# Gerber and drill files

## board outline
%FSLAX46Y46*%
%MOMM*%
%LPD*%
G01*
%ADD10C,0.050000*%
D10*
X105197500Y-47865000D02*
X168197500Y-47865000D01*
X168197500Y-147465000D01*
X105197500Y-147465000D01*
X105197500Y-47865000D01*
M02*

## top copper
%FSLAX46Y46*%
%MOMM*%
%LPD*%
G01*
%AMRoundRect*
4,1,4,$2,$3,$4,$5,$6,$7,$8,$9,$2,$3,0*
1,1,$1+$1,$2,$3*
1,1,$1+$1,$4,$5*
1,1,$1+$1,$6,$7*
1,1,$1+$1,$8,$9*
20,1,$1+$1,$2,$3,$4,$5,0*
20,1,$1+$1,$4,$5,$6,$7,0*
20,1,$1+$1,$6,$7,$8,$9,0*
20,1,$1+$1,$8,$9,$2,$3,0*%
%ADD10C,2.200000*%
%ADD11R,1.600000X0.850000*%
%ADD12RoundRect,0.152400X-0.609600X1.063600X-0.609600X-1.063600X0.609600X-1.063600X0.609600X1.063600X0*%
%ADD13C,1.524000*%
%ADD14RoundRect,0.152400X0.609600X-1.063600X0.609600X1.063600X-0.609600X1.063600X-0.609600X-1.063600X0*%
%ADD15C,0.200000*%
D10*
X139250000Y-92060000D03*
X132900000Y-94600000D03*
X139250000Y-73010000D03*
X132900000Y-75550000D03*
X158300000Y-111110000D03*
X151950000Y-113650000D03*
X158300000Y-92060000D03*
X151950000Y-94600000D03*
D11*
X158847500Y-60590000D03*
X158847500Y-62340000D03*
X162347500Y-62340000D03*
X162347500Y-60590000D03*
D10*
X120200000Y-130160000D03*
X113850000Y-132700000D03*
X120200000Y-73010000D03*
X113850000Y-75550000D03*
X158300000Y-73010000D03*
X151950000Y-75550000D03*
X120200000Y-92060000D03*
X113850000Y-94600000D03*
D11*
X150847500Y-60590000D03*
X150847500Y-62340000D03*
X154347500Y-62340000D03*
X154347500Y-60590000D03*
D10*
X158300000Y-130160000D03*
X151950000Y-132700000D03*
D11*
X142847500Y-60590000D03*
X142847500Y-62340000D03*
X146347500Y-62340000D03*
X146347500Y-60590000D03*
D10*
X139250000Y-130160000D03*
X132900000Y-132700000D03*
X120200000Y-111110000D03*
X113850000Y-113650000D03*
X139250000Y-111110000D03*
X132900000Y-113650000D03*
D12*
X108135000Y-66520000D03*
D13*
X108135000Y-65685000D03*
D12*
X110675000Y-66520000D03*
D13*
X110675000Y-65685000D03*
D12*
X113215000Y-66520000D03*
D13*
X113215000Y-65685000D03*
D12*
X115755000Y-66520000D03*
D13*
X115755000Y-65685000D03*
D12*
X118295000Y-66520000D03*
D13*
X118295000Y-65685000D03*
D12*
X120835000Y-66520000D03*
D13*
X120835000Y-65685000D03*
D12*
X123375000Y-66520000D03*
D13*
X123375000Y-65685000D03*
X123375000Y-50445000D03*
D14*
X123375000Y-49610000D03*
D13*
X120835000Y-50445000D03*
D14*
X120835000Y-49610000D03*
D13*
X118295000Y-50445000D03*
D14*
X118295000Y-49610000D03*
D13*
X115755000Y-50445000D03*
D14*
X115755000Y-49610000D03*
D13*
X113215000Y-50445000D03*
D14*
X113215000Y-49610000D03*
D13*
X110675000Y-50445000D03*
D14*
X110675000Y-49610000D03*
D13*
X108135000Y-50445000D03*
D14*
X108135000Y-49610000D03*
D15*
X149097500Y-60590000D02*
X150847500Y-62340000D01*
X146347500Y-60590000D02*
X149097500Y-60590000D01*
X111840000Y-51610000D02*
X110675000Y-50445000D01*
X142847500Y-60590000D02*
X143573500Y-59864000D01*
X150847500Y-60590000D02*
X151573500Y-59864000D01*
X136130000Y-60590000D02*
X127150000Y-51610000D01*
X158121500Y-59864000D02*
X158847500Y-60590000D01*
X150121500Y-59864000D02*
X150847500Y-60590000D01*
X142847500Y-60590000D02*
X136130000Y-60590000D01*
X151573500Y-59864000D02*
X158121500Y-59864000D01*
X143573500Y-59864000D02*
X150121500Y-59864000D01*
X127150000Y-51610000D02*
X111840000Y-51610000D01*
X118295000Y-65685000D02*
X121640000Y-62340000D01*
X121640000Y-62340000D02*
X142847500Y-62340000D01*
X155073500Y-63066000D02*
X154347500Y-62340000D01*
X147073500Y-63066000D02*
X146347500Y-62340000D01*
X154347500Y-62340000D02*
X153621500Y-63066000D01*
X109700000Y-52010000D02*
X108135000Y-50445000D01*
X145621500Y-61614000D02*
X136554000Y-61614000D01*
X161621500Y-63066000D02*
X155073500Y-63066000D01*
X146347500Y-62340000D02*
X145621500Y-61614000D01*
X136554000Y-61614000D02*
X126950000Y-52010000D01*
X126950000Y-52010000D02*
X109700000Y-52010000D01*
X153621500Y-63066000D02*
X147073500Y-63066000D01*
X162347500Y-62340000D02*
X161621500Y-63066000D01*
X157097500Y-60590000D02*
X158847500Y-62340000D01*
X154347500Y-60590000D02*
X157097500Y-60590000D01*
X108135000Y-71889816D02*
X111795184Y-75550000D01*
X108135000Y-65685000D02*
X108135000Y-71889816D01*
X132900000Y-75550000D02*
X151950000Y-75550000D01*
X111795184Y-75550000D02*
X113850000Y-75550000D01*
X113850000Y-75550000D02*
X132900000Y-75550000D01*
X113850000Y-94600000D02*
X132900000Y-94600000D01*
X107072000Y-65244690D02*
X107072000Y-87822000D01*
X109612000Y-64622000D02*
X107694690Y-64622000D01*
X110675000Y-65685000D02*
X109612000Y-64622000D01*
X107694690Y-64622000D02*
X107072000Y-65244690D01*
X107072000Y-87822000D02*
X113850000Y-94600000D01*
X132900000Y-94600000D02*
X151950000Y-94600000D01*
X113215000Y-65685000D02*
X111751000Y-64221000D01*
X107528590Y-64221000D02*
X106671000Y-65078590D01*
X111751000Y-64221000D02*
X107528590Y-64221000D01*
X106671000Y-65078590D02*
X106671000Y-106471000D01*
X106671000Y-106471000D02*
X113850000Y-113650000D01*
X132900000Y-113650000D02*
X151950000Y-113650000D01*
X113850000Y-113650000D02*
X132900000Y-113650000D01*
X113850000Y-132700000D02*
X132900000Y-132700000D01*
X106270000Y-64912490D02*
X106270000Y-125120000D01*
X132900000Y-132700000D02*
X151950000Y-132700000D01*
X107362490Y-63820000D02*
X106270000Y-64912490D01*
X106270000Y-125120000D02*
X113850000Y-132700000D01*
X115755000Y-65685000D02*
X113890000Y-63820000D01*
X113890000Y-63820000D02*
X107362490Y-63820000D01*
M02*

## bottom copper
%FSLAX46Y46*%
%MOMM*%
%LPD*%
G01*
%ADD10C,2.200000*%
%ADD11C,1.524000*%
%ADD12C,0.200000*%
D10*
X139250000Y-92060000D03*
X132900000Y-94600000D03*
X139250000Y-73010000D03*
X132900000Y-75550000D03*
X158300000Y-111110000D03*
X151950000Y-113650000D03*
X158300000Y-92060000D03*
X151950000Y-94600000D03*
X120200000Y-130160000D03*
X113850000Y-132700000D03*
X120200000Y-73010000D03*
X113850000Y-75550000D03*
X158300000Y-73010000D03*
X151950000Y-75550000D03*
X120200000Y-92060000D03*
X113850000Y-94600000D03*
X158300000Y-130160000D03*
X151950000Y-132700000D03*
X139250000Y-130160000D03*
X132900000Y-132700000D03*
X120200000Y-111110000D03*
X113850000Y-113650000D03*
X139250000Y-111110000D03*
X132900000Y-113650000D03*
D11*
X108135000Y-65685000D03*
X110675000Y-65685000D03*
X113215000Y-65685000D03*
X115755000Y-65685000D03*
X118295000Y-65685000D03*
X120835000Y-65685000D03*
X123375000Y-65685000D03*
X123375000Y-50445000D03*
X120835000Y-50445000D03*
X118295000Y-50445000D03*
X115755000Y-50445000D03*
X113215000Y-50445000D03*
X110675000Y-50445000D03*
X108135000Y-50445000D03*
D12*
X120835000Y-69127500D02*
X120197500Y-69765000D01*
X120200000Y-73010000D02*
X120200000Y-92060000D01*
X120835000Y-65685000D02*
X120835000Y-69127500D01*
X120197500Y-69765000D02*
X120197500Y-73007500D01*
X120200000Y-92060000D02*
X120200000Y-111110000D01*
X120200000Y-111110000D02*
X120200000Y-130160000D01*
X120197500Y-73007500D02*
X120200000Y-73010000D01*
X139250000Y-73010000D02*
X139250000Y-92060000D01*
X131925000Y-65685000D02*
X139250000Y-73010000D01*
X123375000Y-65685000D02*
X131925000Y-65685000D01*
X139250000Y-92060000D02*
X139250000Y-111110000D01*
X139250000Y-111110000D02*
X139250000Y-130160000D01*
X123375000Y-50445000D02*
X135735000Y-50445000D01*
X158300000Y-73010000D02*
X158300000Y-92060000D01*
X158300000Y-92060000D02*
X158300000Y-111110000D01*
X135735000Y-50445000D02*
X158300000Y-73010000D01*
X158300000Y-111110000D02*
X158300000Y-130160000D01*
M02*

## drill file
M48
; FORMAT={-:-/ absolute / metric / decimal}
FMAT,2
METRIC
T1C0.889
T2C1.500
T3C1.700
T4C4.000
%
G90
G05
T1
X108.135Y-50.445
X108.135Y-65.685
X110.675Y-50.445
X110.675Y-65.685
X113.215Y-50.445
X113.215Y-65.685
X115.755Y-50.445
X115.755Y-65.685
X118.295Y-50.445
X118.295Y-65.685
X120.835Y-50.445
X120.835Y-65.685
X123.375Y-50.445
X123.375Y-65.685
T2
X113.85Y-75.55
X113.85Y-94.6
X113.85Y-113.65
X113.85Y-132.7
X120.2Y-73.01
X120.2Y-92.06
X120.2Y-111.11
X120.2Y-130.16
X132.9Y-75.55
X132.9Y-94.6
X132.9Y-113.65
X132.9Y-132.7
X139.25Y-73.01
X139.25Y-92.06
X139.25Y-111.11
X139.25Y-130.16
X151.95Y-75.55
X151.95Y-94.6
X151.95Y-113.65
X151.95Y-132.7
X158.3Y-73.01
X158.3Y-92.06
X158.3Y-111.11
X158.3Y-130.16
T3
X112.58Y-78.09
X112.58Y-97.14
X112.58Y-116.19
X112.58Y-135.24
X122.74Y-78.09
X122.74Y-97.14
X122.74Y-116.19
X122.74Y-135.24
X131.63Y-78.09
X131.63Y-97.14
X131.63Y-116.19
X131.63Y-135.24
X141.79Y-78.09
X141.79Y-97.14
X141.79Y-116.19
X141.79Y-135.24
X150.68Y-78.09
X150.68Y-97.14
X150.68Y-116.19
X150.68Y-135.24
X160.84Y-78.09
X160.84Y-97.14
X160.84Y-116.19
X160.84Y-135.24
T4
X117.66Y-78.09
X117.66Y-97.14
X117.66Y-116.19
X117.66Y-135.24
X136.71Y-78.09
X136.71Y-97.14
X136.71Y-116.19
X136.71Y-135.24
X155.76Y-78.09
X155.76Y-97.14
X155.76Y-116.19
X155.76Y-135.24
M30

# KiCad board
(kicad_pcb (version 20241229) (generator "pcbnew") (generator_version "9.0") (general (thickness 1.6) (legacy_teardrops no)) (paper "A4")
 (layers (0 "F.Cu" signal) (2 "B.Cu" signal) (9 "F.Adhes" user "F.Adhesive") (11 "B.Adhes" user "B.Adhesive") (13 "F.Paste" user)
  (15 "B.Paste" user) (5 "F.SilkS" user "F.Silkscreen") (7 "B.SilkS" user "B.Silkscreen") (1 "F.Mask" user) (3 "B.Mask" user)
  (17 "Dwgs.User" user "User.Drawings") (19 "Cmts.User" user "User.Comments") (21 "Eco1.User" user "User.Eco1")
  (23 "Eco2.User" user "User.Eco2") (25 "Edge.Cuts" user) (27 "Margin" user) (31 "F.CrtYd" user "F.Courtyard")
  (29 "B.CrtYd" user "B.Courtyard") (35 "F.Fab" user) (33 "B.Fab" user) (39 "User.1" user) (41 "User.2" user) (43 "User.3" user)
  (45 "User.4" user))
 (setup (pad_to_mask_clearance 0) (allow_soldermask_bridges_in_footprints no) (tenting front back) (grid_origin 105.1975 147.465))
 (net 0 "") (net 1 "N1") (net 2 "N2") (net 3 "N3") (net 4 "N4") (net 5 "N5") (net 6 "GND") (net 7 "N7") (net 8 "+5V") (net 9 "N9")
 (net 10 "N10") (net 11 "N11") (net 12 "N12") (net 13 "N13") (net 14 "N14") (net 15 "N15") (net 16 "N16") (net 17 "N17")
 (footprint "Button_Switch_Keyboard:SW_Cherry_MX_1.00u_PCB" (layer "F.Cu") (at 139.25 92.06)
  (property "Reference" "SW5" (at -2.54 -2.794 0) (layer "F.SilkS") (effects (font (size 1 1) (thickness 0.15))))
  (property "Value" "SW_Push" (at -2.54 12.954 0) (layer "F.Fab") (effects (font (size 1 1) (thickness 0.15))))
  (pad "" np_thru_hole circle (at -7.62 5.08) (size 1.7 1.7) (drill 1.7) (layers "*.Cu" "*.Mask"))
  (pad "" np_thru_hole circle (at -2.54 5.08) (size 4 4) (drill 4) (layers "*.Cu" "*.Mask"))
  (pad "" np_thru_hole circle (at 2.54 5.08) (size 1.7 1.7) (drill 1.7) (layers "*.Cu" "*.Mask"))
  (pad "1" thru_hole circle (at 0 0) (size 2.2 2.2) (drill 1.5) (layers "*.Cu" "*.Mask") (remove_unused_layers no) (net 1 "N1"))
  (pad "2" thru_hole circle (at -6.35 2.54) (size 2.2 2.2) (drill 1.5) (layers "*.Cu" "*.Mask") (remove_unused_layers no) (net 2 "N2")))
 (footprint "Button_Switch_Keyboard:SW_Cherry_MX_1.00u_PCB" (layer "F.Cu") (at 139.25 73.01)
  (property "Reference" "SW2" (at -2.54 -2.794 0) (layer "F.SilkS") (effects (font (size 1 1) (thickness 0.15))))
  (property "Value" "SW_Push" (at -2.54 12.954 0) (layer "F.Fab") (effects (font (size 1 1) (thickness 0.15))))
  (pad "" np_thru_hole circle (at -7.62 5.08) (size 1.7 1.7) (drill 1.7) (layers "*.Cu" "*.Mask"))
  (pad "" np_thru_hole circle (at -2.54 5.08) (size 4 4) (drill 4) (layers "*.Cu" "*.Mask"))
  (pad "" np_thru_hole circle (at 2.54 5.08) (size 1.7 1.7) (drill 1.7) (layers "*.Cu" "*.Mask"))
  (pad "1" thru_hole circle (at 0 0) (size 2.2 2.2) (drill 1.5) (layers "*.Cu" "*.Mask") (remove_unused_layers no) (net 1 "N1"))
  (pad "2" thru_hole circle (at -6.35 2.54) (size 2.2 2.2) (drill 1.5) (layers "*.Cu" "*.Mask") (remove_unused_layers no) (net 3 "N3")))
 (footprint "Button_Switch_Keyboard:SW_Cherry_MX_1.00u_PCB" (layer "F.Cu") (at 158.3 111.11)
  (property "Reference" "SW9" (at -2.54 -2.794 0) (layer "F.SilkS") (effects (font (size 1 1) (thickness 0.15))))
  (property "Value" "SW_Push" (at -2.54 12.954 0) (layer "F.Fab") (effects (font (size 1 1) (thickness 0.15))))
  (pad "" np_thru_hole circle (at -7.62 5.08) (size 1.7 1.7) (drill 1.7) (layers "*.Cu" "*.Mask"))
  (pad "" np_thru_hole circle (at -2.54 5.08) (size 4 4) (drill 4) (layers "*.Cu" "*.Mask"))
  (pad "" np_thru_hole circle (at 2.54 5.08) (size 1.7 1.7) (drill 1.7) (layers "*.Cu" "*.Mask"))
  (pad "1" thru_hole circle (at 0 0) (size 2.2 2.2) (drill 1.5) (layers "*.Cu" "*.Mask") (remove_unused_layers no) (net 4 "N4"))
  (pad "2" thru_hole circle (at -6.35 2.54) (size 2.2 2.2) (drill 1.5) (layers "*.Cu" "*.Mask") (remove_unused_layers no) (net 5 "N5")))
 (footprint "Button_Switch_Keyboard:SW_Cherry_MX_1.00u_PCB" (layer "F.Cu") (at 158.3 92.06)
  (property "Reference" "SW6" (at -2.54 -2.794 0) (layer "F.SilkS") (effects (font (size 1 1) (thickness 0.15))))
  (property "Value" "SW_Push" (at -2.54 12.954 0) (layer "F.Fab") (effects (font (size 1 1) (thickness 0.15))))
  (pad "" np_thru_hole circle (at -7.62 5.08) (size 1.7 1.7) (drill 1.7) (layers "*.Cu" "*.Mask"))
  (pad "" np_thru_hole circle (at -2.54 5.08) (size 4 4) (drill 4) (layers "*.Cu" "*.Mask"))
  (pad "" np_thru_hole circle (at 2.54 5.08) (size 1.7 1.7) (drill 1.7) (layers "*.Cu" "*.Mask"))
  (pad "1" thru_hole circle (at 0 0) (size 2.2 2.2) (drill 1.5) (layers "*.Cu" "*.Mask") (remove_unused_layers no) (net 4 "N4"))
  (pad "2" thru_hole circle (at -6.35 2.54) (size 2.2 2.2) (drill 1.5) (layers "*.Cu" "*.Mask") (remove_unused_layers no) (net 2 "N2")))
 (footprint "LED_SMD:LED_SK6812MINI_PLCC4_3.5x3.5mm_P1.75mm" (layer "F.Cu") (at 160.5975 61.465)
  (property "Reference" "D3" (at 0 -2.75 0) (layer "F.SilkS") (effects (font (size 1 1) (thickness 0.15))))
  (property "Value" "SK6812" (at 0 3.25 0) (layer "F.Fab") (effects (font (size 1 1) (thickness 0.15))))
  (pad "1" smd rect (at -1.75 -0.875) (size 1.6 0.85) (layers "F.Cu" "F.Mask" "F.Paste") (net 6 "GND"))
  (pad "2" smd rect (at -1.75 0.875) (size 1.6 0.85) (layers "F.Cu" "F.Mask" "F.Paste") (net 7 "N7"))
  (pad "3" smd rect (at 1.75 0.875) (size 1.6 0.85) (layers "F.Cu" "F.Mask" "F.Paste") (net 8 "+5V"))
  (pad "4" smd rect (at 1.75 -0.875) (size 1.6 0.85) (layers "F.Cu" "F.Mask" "F.Paste") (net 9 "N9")))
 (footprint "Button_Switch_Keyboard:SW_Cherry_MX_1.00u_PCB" (layer "F.Cu") (at 120.2 130.16)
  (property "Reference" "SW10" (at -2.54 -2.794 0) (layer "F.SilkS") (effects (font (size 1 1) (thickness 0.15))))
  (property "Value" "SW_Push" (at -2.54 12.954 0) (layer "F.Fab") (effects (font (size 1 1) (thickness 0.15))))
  (pad "" np_thru_hole circle (at -7.62 5.08) (size 1.7 1.7) (drill 1.7) (layers "*.Cu" "*.Mask"))
  (pad "" np_thru_hole circle (at -2.54 5.08) (size 4 4) (drill 4) (layers "*.Cu" "*.Mask"))
  (pad "" np_thru_hole circle (at 2.54 5.08) (size 1.7 1.7) (drill 1.7) (layers "*.Cu" "*.Mask"))
  (pad "1" thru_hole circle (at 0 0) (size 2.2 2.2) (drill 1.5) (layers "*.Cu" "*.Mask") (remove_unused_layers no) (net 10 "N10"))
  (pad "2" thru_hole circle (at -6.35 2.54) (size 2.2 2.2) (drill 1.5) (layers "*.Cu" "*.Mask") (remove_unused_layers no) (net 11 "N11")))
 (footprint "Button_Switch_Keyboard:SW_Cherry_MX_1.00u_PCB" (layer "F.Cu") (at 120.2 73.01)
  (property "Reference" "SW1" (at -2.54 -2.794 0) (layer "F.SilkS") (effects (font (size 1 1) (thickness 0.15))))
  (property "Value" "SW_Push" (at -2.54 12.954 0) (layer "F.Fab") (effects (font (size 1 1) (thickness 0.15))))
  (pad "" np_thru_hole circle (at -7.62 5.08) (size 1.7 1.7) (drill 1.7) (layers "*.Cu" "*.Mask"))
  (pad "" np_thru_hole circle (at -2.54 5.08) (size 4 4) (drill 4) (layers "*.Cu" "*.Mask"))
  (pad "" np_thru_hole circle (at 2.54 5.08) (size 1.7 1.7) (drill 1.7) (layers "*.Cu" "*.Mask"))
  (pad "1" thru_hole circle (at 0 0) (size 2.2 2.2) (drill 1.5) (layers "*.Cu" "*.Mask") (remove_unused_layers no) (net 10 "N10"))
  (pad "2" thru_hole circle (at -6.35 2.54) (size 2.2 2.2) (drill 1.5) (layers "*.Cu" "*.Mask") (remove_unused_layers no) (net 3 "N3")))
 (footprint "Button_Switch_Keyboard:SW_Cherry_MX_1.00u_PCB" (layer "F.Cu") (at 158.3 73.01)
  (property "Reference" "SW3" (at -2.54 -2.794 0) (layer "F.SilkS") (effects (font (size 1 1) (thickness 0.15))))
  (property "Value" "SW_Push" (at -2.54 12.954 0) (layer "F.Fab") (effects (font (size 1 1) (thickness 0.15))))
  (pad "" np_thru_hole circle (at -7.62 5.08) (size 1.7 1.7) (drill 1.7) (layers "*.Cu" "*.Mask"))
  (pad "" np_thru_hole circle (at -2.54 5.08) (size 4 4) (drill 4) (layers "*.Cu" "*.Mask"))
  (pad "" np_thru_hole circle (at 2.54 5.08) (size 1.7 1.7) (drill 1.7) (layers "*.Cu" "*.Mask"))
  (pad "1" thru_hole circle (at 0 0) (size 2.2 2.2) (drill 1.5) (layers "*.Cu" "*.Mask") (remove_unused_layers no) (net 4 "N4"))
  (pad "2" thru_hole circle (at -6.35 2.54) (size 2.2 2.2) (drill 1.5) (layers "*.Cu" "*.Mask") (remove_unused_layers no) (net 3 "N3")))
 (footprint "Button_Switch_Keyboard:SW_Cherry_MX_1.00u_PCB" (layer "F.Cu") (at 120.2 92.06)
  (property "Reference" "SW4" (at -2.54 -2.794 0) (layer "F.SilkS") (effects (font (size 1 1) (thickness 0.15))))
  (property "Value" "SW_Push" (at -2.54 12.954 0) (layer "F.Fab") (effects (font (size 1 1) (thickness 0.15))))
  (pad "" np_thru_hole circle (at -7.62 5.08) (size 1.7 1.7) (drill 1.7) (layers "*.Cu" "*.Mask"))
  (pad "" np_thru_hole circle (at -2.54 5.08) (size 4 4) (drill 4) (layers "*.Cu" "*.Mask"))
  (pad "" np_thru_hole circle (at 2.54 5.08) (size 1.7 1.7) (drill 1.7) (layers "*.Cu" "*.Mask"))
  (pad "1" thru_hole circle (at 0 0) (size 2.2 2.2) (drill 1.5) (layers "*.Cu" "*.Mask") (remove_unused_layers no) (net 10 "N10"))
  (pad "2" thru_hole circle (at -6.35 2.54) (size 2.2 2.2) (drill 1.5) (layers "*.Cu" "*.Mask") (remove_unused_layers no) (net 2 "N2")))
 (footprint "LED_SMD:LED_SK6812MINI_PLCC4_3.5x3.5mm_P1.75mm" (layer "F.Cu") (at 152.5975 61.465)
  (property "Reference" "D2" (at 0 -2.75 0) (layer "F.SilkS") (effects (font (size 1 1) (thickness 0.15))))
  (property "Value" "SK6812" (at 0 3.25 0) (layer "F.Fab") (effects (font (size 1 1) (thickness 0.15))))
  (pad "1" smd rect (at -1.75 -0.875) (size 1.6 0.85) (layers "F.Cu" "F.Mask" "F.Paste") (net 6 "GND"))
  (pad "2" smd rect (at -1.75 0.875) (size 1.6 0.85) (layers "F.Cu" "F.Mask" "F.Paste") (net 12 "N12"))
  (pad "3" smd rect (at 1.75 0.875) (size 1.6 0.85) (layers "F.Cu" "F.Mask" "F.Paste") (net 8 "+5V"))
  (pad "4" smd rect (at 1.75 -0.875) (size 1.6 0.85) (layers "F.Cu" "F.Mask" "F.Paste") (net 7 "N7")))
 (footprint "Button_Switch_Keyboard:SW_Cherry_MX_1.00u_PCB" (layer "F.Cu") (at 158.3 130.16)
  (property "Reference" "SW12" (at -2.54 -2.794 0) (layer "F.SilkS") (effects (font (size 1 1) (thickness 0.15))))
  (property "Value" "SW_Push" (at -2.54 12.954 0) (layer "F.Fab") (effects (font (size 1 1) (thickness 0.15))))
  (pad "" np_thru_hole circle (at -7.62 5.08) (size 1.7 1.7) (drill 1.7) (layers "*.Cu" "*.Mask"))
  (pad "" np_thru_hole circle (at -2.54 5.08) (size 4 4) (drill 4) (layers "*.Cu" "*.Mask"))
  (pad "" np_thru_hole circle (at 2.54 5.08) (size 1.7 1.7) (drill 1.7) (layers "*.Cu" "*.Mask"))
  (pad "1" thru_hole circle (at 0 0) (size 2.2 2.2) (drill 1.5) (layers "*.Cu" "*.Mask") (remove_unused_layers no) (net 4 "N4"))
  (pad "2" thru_hole circle (at -6.35 2.54) (size 2.2 2.2) (drill 1.5) (layers "*.Cu" "*.Mask") (remove_unused_layers no) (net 11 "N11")))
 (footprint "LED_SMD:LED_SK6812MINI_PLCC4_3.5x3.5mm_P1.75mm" (layer "F.Cu") (at 144.5975 61.465)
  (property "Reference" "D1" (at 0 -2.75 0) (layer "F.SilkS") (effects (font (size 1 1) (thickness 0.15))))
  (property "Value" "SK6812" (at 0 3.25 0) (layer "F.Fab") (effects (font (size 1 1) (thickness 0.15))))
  (pad "1" smd rect (at -1.75 -0.875) (size 1.6 0.85) (layers "F.Cu" "F.Mask" "F.Paste") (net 6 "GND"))
  (pad "2" smd rect (at -1.75 0.875) (size 1.6 0.85) (layers "F.Cu" "F.Mask" "F.Paste") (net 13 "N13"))
  (pad "3" smd rect (at 1.75 0.875) (size 1.6 0.85) (layers "F.Cu" "F.Mask" "F.Paste") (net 8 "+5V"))
  (pad "4" smd rect (at 1.75 -0.875) (size 1.6 0.85) (layers "F.Cu" "F.Mask" "F.Paste") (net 12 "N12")))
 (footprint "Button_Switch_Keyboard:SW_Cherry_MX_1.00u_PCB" (layer "F.Cu") (at 139.25 130.16)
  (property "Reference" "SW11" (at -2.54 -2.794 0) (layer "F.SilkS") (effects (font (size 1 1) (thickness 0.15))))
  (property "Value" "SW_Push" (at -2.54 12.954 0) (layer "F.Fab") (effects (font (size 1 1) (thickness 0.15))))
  (pad "" np_thru_hole circle (at -7.62 5.08) (size 1.7 1.7) (drill 1.7) (layers "*.Cu" "*.Mask"))
  (pad "" np_thru_hole circle (at -2.54 5.08) (size 4 4) (drill 4) (layers "*.Cu" "*.Mask"))
  (pad "" np_thru_hole circle (at 2.54 5.08) (size 1.7 1.7) (drill 1.7) (layers "*.Cu" "*.Mask"))
  (pad "1" thru_hole circle (at 0 0) (size 2.2 2.2) (drill 1.5) (layers "*.Cu" "*.Mask") (remove_unused_layers no) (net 1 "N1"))
  (pad "2" thru_hole circle (at -6.35 2.54) (size 2.2 2.2) (drill 1.5) (layers "*.Cu" "*.Mask") (remove_unused_layers no) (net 11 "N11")))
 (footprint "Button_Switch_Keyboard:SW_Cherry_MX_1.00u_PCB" (layer "F.Cu") (at 120.2 111.11)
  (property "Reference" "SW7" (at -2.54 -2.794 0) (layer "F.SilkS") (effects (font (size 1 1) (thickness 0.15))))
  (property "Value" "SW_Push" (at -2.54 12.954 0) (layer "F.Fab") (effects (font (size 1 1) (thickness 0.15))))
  (pad "" np_thru_hole circle (at -7.62 5.08) (size 1.7 1.7) (drill 1.7) (layers "*.Cu" "*.Mask"))
  (pad "" np_thru_hole circle (at -2.54 5.08) (size 4 4) (drill 4) (layers "*.Cu" "*.Mask"))
  (pad "" np_thru_hole circle (at 2.54 5.08) (size 1.7 1.7) (drill 1.7) (layers "*.Cu" "*.Mask"))
  (pad "1" thru_hole circle (at 0 0) (size 2.2 2.2) (drill 1.5) (layers "*.Cu" "*.Mask") (remove_unused_layers no) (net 10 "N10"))
  (pad "2" thru_hole circle (at -6.35 2.54) (size 2.2 2.2) (drill 1.5) (layers "*.Cu" "*.Mask") (remove_unused_layers no) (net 5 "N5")))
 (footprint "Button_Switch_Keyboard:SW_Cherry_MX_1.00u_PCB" (layer "F.Cu") (at 139.25 111.11)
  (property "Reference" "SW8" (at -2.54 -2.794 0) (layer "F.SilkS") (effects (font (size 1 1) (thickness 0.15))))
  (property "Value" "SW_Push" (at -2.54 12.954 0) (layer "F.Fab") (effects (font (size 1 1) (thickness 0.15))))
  (pad "" np_thru_hole circle (at -7.62 5.08) (size 1.7 1.7) (drill 1.7) (layers "*.Cu" "*.Mask"))
  (pad "" np_thru_hole circle (at -2.54 5.08) (size 4 4) (drill 4) (layers "*.Cu" "*.Mask"))
  (pad "" np_thru_hole circle (at 2.54 5.08) (size 1.7 1.7) (drill 1.7) (layers "*.Cu" "*.Mask"))
  (pad "1" thru_hole circle (at 0 0) (size 2.2 2.2) (drill 1.5) (layers "*.Cu" "*.Mask") (remove_unused_layers no) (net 1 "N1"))
  (pad "2" thru_hole circle (at -6.35 2.54) (size 2.2 2.2) (drill 1.5) (layers "*.Cu" "*.Mask") (remove_unused_layers no) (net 5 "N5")))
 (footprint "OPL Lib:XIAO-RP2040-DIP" (layer "F.Cu") (at 115.755 58.065 90)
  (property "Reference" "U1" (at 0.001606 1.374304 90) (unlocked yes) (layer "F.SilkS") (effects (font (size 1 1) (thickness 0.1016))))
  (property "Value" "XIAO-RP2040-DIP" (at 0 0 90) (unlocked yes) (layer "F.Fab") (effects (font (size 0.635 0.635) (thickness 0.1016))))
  (pad "1" smd roundrect (at -8.455 -7.62 270) (size 2.432 1.524) (layers "F.Cu" "F.Mask") (roundrect_rratio 0.1) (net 3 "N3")
   (thermal_bridge_angle 45))
  (pad "1" thru_hole circle (at -7.62 -7.62 270) (size 1.524 1.524) (drill 0.889) (layers "*.Cu" "*.Mask") (remove_unused_layers no)
   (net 3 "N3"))
  (pad "2" smd roundrect (at -8.455 -5.08 270) (size 2.432 1.524) (layers "F.Cu" "F.Mask") (roundrect_rratio 0.1) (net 2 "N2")
   (thermal_bridge_angle 45))
  (pad "2" thru_hole circle (at -7.62 -5.08 270) (size 1.524 1.524) (drill 0.889) (layers "*.Cu" "*.Mask") (remove_unused_layers no)
   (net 2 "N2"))
  (pad "3" smd roundrect (at -8.455 -2.54 270) (size 2.432 1.524) (layers "F.Cu" "F.Mask") (roundrect_rratio 0.1) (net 5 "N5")
   (thermal_bridge_angle 45))
  (pad "3" thru_hole circle (at -7.62 -2.54 270) (size 1.524 1.524) (drill 0.889) (layers "*.Cu" "*.Mask") (remove_unused_layers no)
   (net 5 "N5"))
  (pad "4" smd roundrect (at -8.455 0 270) (size 2.432 1.524) (layers "F.Cu" "F.Mask") (roundrect_rratio 0.1) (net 11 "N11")
   (thermal_bridge_angle 45))
  (pad "4" thru_hole circle (at -7.62 0 270) (size 1.524 1.524) (drill 0.889) (layers "*.Cu" "*.Mask") (remove_unused_layers no)
   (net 11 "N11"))
  (pad "5" smd roundrect (at -8.455 2.54 270) (size 2.432 1.524) (layers "F.Cu" "F.Mask") (roundrect_rratio 0.1) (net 13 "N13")
   (thermal_bridge_angle 45))
  (pad "5" thru_hole circle (at -7.62 2.54 270) (size 1.524 1.524) (drill 0.889) (layers "*.Cu" "*.Mask") (remove_unused_layers no)
   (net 13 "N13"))
  (pad "6" smd roundrect (at -8.455 5.08 270) (size 2.432 1.524) (layers "F.Cu" "F.Mask") (roundrect_rratio 0.1) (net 10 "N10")
   (thermal_bridge_angle 45))
  (pad "6" thru_hole circle (at -7.62 5.08 270) (size 1.524 1.524) (drill 0.889) (layers "*.Cu" "*.Mask") (remove_unused_layers no)
   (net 10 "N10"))
  (pad "7" smd roundrect (at -8.455 7.62 270) (size 2.432 1.524) (layers "F.Cu" "F.Mask") (roundrect_rratio 0.1) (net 1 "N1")
   (thermal_bridge_angle 45))
  (pad "7" thru_hole circle (at -7.62 7.62 270) (size 1.524 1.524) (drill 0.889) (layers "*.Cu" "*.Mask") (remove_unused_layers no)
   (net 1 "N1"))
  (pad "8" thru_hole circle (at 7.62 7.62 90) (size 1.524 1.524) (drill 0.889) (layers "*.Cu" "*.Mask") (remove_unused_layers no)
   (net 4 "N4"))
  (pad "8" smd roundrect (at 8.455 7.62 90) (size 2.432 1.524) (layers "F.Cu" "F.Mask") (roundrect_rratio 0.1) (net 4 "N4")
   (thermal_bridge_angle 45))
  (pad "9" thru_hole circle (at 7.62 5.08 90) (size 1.524 1.524) (drill 0.889) (layers "*.Cu" "*.Mask") (remove_unused_layers no)
   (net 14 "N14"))
  (pad "9" smd roundrect (at 8.455 5.08 90) (size 2.432 1.524) (layers "F.Cu" "F.Mask") (roundrect_rratio 0.1) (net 14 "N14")
   (thermal_bridge_angle 45))
  (pad "10" thru_hole circle (at 7.62 2.54 90) (size 1.524 1.524) (drill 0.889) (layers "*.Cu" "*.Mask") (remove_unused_layers no)
   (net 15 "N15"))
  (pad "10" smd roundrect (at 8.455 2.54 90) (size 2.432 1.524) (layers "F.Cu" "F.Mask") (roundrect_rratio 0.1) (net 15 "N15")
   (thermal_bridge_angle 45))
  (pad "11" thru_hole circle (at 7.62 0 90) (size 1.524 1.524) (drill 0.889) (layers "*.Cu" "*.Mask") (remove_unused_layers no)
   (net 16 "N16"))
  (pad "11" smd roundrect (at 8.455 0 90) (size 2.432 1.524) (layers "F.Cu" "F.Mask") (roundrect_rratio 0.1) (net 16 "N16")
   (thermal_bridge_angle 45))
  (pad "12" thru_hole circle (at 7.62 -2.54 90) (size 1.524 1.524) (drill 0.889) (layers "*.Cu" "*.Mask") (remove_unused_layers no)
   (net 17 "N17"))
  (pad "12" smd roundrect (at 8.455 -2.54 90) (size 2.432 1.524) (layers "F.Cu" "F.Mask") (roundrect_rratio 0.1) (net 17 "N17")
   (thermal_bridge_angle 45))
  (pad "13" thru_hole circle (at 7.62 -5.08 90) (size 1.524 1.524) (drill 0.889) (layers "*.Cu" "*.Mask") (remove_unused_layers no)
   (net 6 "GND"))
  (pad "13" smd roundrect (at 8.455 -5.08 90) (size 2.432 1.524) (layers "F.Cu" "F.Mask") (roundrect_rratio 0.1) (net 6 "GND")
   (thermal_bridge_angle 45))
  (pad "14" thru_hole circle (at 7.62 -7.62 90) (size 1.524 1.524) (drill 0.889) (layers "*.Cu" "*.Mask") (remove_unused_layers no)
   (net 8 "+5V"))
  (pad "14" smd roundrect (at 8.455 -7.62 90) (size 2.432 1.524) (layers "F.Cu" "F.Mask") (roundrect_rratio 0.1) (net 8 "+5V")
   (thermal_bridge_angle 45)))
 (gr_rect (start 105.1975 47.865) (end 168.1975 147.465) (stroke (width 0.05) (type default)) (fill no) (layer "Edge.Cuts"))
 (segment (start 149.0975 60.59) (end 150.8475 62.34) (width 0.2) (layer "F.Cu") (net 12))
 (segment (start 146.3475 60.59) (end 149.0975 60.59) (width 0.2) (layer "F.Cu") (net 12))
 (segment (start 111.84 51.61) (end 110.675 50.445) (width 0.2) (layer "F.Cu") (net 6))
 (segment (start 142.8475 60.59) (end 143.5735 59.864) (width 0.2) (layer "F.Cu") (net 6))
 (segment (start 150.8475 60.59) (end 151.5735 59.864) (width 0.2) (layer "F.Cu") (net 6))
 (segment (start 136.13 60.59) (end 127.15 51.61) (width 0.2) (layer "F.Cu") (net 6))
 (segment (start 158.1215 59.864) (end 158.8475 60.59) (width 0.2) (layer "F.Cu") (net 6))
 (segment (start 150.1215 59.864) (end 150.8475 60.59) (width 0.2) (layer "F.Cu") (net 6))
 (segment (start 142.8475 60.59) (end 136.13 60.59) (width 0.2) (layer "F.Cu") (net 6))
 (segment (start 151.5735 59.864) (end 158.1215 59.864) (width 0.2) (layer "F.Cu") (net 6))
 (segment (start 143.5735 59.864) (end 150.1215 59.864) (width 0.2) (layer "F.Cu") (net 6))
 (segment (start 127.15 51.61) (end 111.84 51.61) (width 0.2) (layer "F.Cu") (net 6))
 (segment (start 118.295 65.685) (end 121.64 62.34) (width 0.2) (layer "F.Cu") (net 13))
 (segment (start 121.64 62.34) (end 142.8475 62.34) (width 0.2) (layer "F.Cu") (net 13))
 (segment (start 155.0735 63.066) (end 154.3475 62.34) (width 0.2) (layer "F.Cu") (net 8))
 (segment (start 147.0735 63.066) (end 146.3475 62.34) (width 0.2) (layer "F.Cu") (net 8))
 (segment (start 154.3475 62.34) (end 153.6215 63.066) (width 0.2) (layer "F.Cu") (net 8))
 (segment (start 109.7 52.01) (end 108.135 50.445) (width 0.2) (layer "F.Cu") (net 8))
 (segment (start 145.6215 61.614) (end 136.554 61.614) (width 0.2) (layer "F.Cu") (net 8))
 (segment (start 161.6215 63.066) (end 155.0735 63.066) (width 0.2) (layer "F.Cu") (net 8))
 (segment (start 146.3475 62.34) (end 145.6215 61.614) (width 0.2) (layer "F.Cu") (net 8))
 (segment (start 136.554 61.614) (end 126.95 52.01) (width 0.2) (layer "F.Cu") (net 8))
 (segment (start 126.95 52.01) (end 109.7 52.01) (width 0.2) (layer "F.Cu") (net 8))
 (segment (start 153.6215 63.066) (end 147.0735 63.066) (width 0.2) (layer "F.Cu") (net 8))
 (segment (start 162.3475 62.34) (end 161.6215 63.066) (width 0.2) (layer "F.Cu") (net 8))
 (segment (start 157.0975 60.59) (end 158.8475 62.34) (width 0.2) (layer "F.Cu") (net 7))
 (segment (start 154.3475 60.59) (end 157.0975 60.59) (width 0.2) (layer "F.Cu") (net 7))
 (segment (start 108.135 71.889816) (end 111.795184 75.55) (width 0.2) (layer "F.Cu") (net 3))
 (segment (start 108.135 65.685) (end 108.135 71.889816) (width 0.2) (layer "F.Cu") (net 3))
 (segment (start 132.9 75.55) (end 151.95 75.55) (width 0.2) (layer "F.Cu") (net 3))
 (segment (start 111.795184 75.55) (end 113.85 75.55) (width 0.2) (layer "F.Cu") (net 3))
 (segment (start 113.85 75.55) (end 132.9 75.55) (width 0.2) (layer "F.Cu") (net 3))
 (segment (start 120.835 69.1275) (end 120.1975 69.765) (width 0.2) (layer "B.Cu") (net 10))
 (segment (start 120.2 73.01) (end 120.2 92.06) (width 0.2) (layer "B.Cu") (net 10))
 (segment (start 120.835 65.685) (end 120.835 69.1275) (width 0.2) (layer "B.Cu") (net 10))
 (segment (start 120.1975 69.765) (end 120.1975 73.0075) (width 0.2) (layer "B.Cu") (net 10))
 (segment (start 120.2 92.06) (end 120.2 111.11) (width 0.2) (layer "B.Cu") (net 10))
 (segment (start 120.2 111.11) (end 120.2 130.16) (width 0.2) (layer "B.Cu") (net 10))
 (segment (start 120.1975 73.0075) (end 120.2 73.01) (width 0.2) (layer "B.Cu") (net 10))
 (segment (start 139.25 73.01) (end 139.25 92.06) (width 0.2) (layer "B.Cu") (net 1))
 (segment (start 131.925 65.685) (end 139.25 73.01) (width 0.2) (layer "B.Cu") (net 1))
 (segment (start 123.375 65.685) (end 131.925 65.685) (width 0.2) (layer "B.Cu") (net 1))
 (segment (start 139.25 92.06) (end 139.25 111.11) (width 0.2) (layer "B.Cu") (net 1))
 (segment (start 139.25 111.11) (end 139.25 130.16) (width 0.2) (layer "B.Cu") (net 1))
 (segment (start 123.375 50.445) (end 135.735 50.445) (width 0.2) (layer "B.Cu") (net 4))
 (segment (start 158.3 73.01) (end 158.3 92.06) (width 0.2) (layer "B.Cu") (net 4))
 (segment (start 158.3 92.06) (end 158.3 111.11) (width 0.2) (layer "B.Cu") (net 4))
 (segment (start 135.735 50.445) (end 158.3 73.01) (width 0.2) (layer "B.Cu") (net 4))
 (segment (start 158.3 111.11) (end 158.3 130.16) (width 0.2) (layer "B.Cu") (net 4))
 (segment (start 113.85 94.6) (end 132.9 94.6) (width 0.2) (layer "F.Cu") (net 2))
 (segment (start 107.072 65.24469) (end 107.072 87.822) (width 0.2) (layer "F.Cu") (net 2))
 (segment (start 109.612 64.622) (end 107.69469 64.622) (width 0.2) (layer "F.Cu") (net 2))
 (segment (start 110.675 65.685) (end 109.612 64.622) (width 0.2) (layer "F.Cu") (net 2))
 (segment (start 107.69469 64.622) (end 107.072 65.24469) (width 0.2) (layer "F.Cu") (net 2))
 (segment (start 107.072 87.822) (end 113.85 94.6) (width 0.2) (layer "F.Cu") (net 2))
 (segment (start 132.9 94.6) (end 151.95 94.6) (width 0.2) (layer "F.Cu") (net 2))
 (segment (start 113.215 65.685) (end 111.751 64.221) (width 0.2) (layer "F.Cu") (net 5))
 (segment (start 107.52859 64.221) (end 106.671 65.07859) (width 0.2) (layer "F.Cu") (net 5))
 (segment (start 111.751 64.221) (end 107.52859 64.221) (width 0.2) (layer "F.Cu") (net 5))
 (segment (start 106.671 65.07859) (end 106.671 106.471) (width 0.2) (layer "F.Cu") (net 5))
 (segment (start 106.671 106.471) (end 113.85 113.65) (width 0.2) (layer "F.Cu") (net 5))
 (segment (start 132.9 113.65) (end 151.95 113.65) (width 0.2) (layer "F.Cu") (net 5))
 (segment (start 113.85 113.65) (end 132.9 113.65) (width 0.2) (layer "F.Cu") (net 5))
 (segment (start 113.85 132.7) (end 132.9 132.7) (width 0.2) (layer "F.Cu") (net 11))
 (segment (start 106.27 64.91249) (end 106.27 125.12) (width 0.2) (layer "F.Cu") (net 11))
 (segment (start 132.9 132.7) (end 151.95 132.7) (width 0.2) (layer "F.Cu") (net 11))
 (segment (start 107.36249 63.82) (end 106.27 64.91249) (width 0.2) (layer "F.Cu") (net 11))
 (segment (start 106.27 125.12) (end 113.85 132.7) (width 0.2) (layer "F.Cu") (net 11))
 (segment (start 115.755 65.685) (end 113.89 63.82) (width 0.2) (layer "F.Cu") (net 11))
 (segment (start 113.89 63.82) (end 107.36249 63.82) (width 0.2) (layer "F.Cu") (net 11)))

